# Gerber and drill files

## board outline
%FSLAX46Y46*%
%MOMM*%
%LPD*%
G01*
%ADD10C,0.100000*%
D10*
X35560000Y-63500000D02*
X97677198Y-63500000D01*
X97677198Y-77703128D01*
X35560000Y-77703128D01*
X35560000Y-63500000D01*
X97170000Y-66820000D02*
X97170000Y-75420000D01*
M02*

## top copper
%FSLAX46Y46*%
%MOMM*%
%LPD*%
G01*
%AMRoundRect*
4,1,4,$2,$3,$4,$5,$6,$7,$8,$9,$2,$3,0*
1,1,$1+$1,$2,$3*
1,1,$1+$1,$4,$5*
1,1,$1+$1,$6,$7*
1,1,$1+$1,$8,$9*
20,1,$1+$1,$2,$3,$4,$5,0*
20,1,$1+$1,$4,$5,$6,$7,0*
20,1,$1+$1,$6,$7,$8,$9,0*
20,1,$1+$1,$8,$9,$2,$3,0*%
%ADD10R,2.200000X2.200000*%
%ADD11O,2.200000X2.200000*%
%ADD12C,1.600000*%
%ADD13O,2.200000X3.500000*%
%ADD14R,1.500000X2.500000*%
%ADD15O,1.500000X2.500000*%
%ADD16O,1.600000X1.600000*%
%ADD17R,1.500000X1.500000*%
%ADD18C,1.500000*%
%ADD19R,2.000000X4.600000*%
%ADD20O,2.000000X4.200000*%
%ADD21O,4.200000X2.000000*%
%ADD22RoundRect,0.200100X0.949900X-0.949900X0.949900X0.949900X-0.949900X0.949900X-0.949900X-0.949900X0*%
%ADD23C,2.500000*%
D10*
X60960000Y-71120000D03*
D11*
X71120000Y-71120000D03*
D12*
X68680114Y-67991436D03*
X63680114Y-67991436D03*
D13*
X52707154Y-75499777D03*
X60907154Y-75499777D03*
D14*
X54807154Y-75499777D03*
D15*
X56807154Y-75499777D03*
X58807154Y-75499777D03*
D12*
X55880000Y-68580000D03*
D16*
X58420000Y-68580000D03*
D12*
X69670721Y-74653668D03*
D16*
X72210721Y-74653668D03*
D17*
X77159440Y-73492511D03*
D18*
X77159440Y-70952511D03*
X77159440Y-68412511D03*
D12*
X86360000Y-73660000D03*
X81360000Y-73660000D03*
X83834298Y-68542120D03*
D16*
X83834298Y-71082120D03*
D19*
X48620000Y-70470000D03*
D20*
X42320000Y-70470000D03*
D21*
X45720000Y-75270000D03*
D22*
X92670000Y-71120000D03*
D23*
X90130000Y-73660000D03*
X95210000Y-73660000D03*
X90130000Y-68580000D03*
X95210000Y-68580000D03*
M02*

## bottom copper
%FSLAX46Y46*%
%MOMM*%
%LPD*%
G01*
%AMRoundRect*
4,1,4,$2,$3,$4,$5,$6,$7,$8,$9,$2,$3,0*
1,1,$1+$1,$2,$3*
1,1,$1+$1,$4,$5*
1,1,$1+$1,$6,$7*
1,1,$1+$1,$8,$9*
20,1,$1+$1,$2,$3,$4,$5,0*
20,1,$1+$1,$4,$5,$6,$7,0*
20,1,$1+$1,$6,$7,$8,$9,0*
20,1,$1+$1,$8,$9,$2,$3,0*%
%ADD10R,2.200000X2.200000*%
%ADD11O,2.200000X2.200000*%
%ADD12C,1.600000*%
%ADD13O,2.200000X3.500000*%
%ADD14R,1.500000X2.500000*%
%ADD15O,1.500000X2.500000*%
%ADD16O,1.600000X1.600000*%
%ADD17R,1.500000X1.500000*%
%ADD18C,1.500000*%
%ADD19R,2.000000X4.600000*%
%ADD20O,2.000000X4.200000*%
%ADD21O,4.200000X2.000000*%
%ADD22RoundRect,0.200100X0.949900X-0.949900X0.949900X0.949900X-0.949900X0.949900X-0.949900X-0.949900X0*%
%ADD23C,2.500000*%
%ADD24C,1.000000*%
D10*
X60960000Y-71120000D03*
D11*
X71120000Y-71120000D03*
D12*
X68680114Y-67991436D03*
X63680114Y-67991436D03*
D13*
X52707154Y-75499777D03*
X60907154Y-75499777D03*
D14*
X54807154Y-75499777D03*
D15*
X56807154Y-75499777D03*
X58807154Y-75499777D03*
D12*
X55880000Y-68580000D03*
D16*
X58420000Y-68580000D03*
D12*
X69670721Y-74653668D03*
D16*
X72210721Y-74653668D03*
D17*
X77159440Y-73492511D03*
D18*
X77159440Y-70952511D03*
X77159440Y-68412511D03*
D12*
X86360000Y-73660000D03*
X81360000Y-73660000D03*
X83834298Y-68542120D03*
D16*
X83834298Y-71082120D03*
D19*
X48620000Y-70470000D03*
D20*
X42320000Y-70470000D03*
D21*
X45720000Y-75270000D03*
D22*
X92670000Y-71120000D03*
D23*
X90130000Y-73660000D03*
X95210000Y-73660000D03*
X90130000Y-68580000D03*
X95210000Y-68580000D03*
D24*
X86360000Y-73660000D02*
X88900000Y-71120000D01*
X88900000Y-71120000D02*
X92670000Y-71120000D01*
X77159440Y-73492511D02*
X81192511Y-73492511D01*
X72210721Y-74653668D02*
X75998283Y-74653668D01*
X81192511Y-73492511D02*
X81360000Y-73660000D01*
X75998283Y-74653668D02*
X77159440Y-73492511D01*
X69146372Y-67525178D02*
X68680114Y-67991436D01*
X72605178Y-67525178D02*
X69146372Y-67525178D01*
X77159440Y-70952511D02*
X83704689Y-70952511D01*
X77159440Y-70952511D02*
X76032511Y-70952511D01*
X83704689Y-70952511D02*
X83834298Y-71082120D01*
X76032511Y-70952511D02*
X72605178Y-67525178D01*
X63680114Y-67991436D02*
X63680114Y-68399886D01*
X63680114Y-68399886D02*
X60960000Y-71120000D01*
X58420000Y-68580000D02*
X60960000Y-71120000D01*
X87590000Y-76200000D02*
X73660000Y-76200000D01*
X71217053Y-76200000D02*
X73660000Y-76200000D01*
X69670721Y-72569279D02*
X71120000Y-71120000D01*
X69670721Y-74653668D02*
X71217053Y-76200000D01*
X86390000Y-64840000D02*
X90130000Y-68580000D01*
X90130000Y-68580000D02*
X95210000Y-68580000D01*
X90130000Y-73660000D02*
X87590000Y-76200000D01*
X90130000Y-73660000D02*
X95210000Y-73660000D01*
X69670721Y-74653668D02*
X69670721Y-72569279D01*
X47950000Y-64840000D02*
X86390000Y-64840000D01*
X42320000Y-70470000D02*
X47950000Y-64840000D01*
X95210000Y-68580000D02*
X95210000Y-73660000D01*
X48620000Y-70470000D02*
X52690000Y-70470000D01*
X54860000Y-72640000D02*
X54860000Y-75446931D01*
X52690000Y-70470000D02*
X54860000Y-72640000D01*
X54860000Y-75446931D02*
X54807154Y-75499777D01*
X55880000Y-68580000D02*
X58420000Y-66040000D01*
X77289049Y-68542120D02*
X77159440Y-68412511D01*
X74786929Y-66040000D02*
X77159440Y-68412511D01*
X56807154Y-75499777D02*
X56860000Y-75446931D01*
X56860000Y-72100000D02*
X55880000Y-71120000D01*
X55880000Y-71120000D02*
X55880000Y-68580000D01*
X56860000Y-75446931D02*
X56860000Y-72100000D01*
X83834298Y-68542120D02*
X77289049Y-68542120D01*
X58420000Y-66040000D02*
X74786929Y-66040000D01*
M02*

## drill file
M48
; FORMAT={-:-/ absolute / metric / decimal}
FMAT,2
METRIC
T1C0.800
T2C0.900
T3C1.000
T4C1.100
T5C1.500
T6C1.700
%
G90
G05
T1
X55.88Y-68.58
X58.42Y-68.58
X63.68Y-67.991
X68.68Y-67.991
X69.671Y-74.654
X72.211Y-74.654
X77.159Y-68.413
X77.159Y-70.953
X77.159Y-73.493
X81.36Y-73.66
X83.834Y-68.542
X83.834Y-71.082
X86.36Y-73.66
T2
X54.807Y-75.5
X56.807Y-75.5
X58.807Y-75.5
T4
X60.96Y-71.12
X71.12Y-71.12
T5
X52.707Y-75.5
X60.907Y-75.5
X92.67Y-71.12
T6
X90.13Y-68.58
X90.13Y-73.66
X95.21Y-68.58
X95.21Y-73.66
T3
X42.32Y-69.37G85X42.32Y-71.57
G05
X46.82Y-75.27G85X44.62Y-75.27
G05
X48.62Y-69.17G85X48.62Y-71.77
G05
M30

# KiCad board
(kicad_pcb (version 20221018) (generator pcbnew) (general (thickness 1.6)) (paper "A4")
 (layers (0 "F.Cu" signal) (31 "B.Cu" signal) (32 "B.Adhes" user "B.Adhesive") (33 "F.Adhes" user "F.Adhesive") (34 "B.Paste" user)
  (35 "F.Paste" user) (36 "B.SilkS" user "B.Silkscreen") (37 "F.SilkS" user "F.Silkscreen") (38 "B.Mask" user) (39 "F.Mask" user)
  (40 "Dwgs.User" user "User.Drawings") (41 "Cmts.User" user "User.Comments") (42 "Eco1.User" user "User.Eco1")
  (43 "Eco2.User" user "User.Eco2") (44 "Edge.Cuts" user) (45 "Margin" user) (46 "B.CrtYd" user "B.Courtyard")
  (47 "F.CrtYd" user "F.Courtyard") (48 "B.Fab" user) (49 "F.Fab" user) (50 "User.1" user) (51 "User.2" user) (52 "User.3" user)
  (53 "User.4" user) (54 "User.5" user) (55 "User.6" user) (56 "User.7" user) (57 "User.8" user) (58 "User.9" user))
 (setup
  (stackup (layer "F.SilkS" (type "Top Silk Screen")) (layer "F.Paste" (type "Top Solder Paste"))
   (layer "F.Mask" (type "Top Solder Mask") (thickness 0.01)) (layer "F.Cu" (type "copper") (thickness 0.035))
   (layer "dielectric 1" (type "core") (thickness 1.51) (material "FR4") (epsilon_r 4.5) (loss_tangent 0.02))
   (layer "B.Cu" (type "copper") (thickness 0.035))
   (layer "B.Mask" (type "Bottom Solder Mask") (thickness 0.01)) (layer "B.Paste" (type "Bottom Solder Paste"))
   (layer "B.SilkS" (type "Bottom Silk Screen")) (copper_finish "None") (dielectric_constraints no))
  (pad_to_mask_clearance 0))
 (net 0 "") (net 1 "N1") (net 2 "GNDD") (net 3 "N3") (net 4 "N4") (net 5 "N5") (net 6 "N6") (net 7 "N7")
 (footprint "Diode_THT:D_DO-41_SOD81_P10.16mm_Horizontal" (layer "F.Cu") (at 60.96 71.12)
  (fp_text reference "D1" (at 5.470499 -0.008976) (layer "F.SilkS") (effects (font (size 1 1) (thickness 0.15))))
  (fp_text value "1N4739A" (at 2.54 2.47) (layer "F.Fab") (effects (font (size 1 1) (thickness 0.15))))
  (pad "1" thru_hole rect (at 0 0) (size 2.2 2.2) (drill 1.1) (layers "*.Cu" "*.Mask") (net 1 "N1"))
  (pad "2" thru_hole oval (at 10.16 0) (size 2.2 2.2) (drill 1.1) (layers "*.Cu" "*.Mask") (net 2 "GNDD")))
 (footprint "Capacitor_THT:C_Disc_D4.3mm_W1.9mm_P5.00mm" (layer "F.Cu") (at 68.680114 67.991436 180)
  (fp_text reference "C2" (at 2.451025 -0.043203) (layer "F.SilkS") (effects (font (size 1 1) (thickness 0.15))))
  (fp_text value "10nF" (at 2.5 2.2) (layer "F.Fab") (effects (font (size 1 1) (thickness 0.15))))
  (pad "1" thru_hole circle (at 0 0 180) (size 1.6 1.6) (drill 0.8) (layers "*.Cu" "*.Mask") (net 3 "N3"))
  (pad "2" thru_hole circle (at 5 0 180) (size 1.6 1.6) (drill 0.8) (layers "*.Cu" "*.Mask") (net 1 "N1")))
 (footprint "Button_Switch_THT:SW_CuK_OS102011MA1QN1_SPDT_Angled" (layer "F.Cu") (at 54.807154 75.499777)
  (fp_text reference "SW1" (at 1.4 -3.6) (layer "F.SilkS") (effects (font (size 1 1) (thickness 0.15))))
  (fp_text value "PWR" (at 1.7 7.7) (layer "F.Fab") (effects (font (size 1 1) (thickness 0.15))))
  (pad "" thru_hole oval (at -2.1 0) (size 2.2 3.5) (drill 1.5) (layers "*.Cu" "*.Mask"))
  (pad "" thru_hole oval (at 6.1 0) (size 2.2 3.5) (drill 1.5) (layers "*.Cu" "*.Mask"))
  (pad "1" thru_hole rect (at 0 0) (size 1.5 2.5) (drill 0.9) (layers "*.Cu" "*.Mask") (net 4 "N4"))
  (pad "2" thru_hole oval (at 2 0) (size 1.5 2.5) (drill 0.9) (layers "*.Cu" "*.Mask") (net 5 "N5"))
  (pad "3" thru_hole oval (at 4 0) (size 1.5 2.5) (drill 0.9) (layers "*.Cu" "*.Mask")))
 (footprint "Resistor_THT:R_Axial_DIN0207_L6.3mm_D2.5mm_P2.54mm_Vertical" (layer "F.Cu") (at 55.88 68.58)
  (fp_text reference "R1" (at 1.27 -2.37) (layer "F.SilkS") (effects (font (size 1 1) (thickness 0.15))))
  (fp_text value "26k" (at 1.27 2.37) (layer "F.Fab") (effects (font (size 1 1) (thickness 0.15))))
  (pad "1" thru_hole circle (at 0 0) (size 1.6 1.6) (drill 0.8) (layers "*.Cu" "*.Mask") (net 5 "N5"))
  (pad "2" thru_hole oval (at 2.54 0) (size 1.6 1.6) (drill 0.8) (layers "*.Cu" "*.Mask") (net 1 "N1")))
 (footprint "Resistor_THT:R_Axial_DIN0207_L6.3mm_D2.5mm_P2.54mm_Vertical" (layer "F.Cu") (at 69.670721 74.653668)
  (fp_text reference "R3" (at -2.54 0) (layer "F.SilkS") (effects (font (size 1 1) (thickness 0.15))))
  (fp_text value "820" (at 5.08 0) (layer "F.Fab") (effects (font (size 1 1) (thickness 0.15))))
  (pad "1" thru_hole circle (at 0 0) (size 1.6 1.6) (drill 0.8) (layers "*.Cu" "*.Mask") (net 2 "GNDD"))
  (pad "2" thru_hole oval (at 2.54 0) (size 1.6 1.6) (drill 0.8) (layers "*.Cu" "*.Mask") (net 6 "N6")))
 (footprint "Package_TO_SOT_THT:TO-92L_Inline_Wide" (layer "F.Cu") (at 77.15944 73.492511 90)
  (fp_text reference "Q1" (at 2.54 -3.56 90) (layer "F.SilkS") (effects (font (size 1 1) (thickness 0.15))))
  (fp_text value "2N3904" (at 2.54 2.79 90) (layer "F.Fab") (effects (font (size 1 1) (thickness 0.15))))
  (pad "1" thru_hole rect (at 0 0 90) (size 1.5 1.5) (drill 0.8) (layers "*.Cu" "*.Mask") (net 6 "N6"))
  (pad "2" thru_hole circle (at 2.54 0 90) (size 1.5 1.5) (drill 0.8) (layers "*.Cu" "*.Mask") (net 3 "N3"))
  (pad "3" thru_hole circle (at 5.08 0 90) (size 1.5 1.5) (drill 0.8) (layers "*.Cu" "*.Mask") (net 5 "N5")))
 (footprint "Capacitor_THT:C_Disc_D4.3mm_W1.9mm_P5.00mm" (layer "F.Cu") (at 86.36 73.66 180)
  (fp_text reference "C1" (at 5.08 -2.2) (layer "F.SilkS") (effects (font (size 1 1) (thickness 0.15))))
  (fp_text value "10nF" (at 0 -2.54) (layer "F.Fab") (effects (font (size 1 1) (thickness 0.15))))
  (pad "1" thru_hole circle (at 0 0 180) (size 1.6 1.6) (drill 0.8) (layers "*.Cu" "*.Mask") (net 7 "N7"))
  (pad "2" thru_hole circle (at 5 0 180) (size 1.6 1.6) (drill 0.8) (layers "*.Cu" "*.Mask") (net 6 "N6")))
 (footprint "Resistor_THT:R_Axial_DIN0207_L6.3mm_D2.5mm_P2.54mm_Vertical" (layer "F.Cu") (at 83.834298 68.54212 -90)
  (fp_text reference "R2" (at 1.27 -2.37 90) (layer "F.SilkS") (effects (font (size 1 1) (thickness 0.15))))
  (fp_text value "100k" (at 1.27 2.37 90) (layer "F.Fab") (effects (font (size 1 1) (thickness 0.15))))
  (pad "1" thru_hole circle (at 0 0 270) (size 1.6 1.6) (drill 0.8) (layers "*.Cu" "*.Mask") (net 5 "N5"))
  (pad "2" thru_hole oval (at 2.54 0 270) (size 1.6 1.6) (drill 0.8) (layers "*.Cu" "*.Mask") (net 3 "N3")))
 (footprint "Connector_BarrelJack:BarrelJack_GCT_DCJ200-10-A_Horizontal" (layer "F.Cu") (at 48.62 70.47 -90)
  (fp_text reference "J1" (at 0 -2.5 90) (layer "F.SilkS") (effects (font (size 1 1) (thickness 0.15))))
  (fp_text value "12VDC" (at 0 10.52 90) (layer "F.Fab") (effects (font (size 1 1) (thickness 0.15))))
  (pad "1" thru_hole rect (at 0 0 270) (size 4.6 2) (drill oval 3.6 1) (layers "*.Cu" "*.Mask") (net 4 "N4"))
  (pad "2" thru_hole oval (at 0 6.3 270) (size 4.2 2) (drill oval 3.2 1) (layers "*.Cu" "*.Mask") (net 2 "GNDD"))
  (pad "3" thru_hole oval (at 4.8 2.9 270) (size 2 4.2) (drill oval 1 3.2) (layers "*.Cu" "*.Mask")))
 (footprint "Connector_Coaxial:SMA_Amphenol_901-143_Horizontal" (layer "B.Cu") (at 92.67 71.12 90)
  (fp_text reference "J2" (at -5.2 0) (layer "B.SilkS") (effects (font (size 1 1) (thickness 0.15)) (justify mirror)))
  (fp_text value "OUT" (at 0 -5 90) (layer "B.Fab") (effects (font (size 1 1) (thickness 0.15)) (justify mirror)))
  (fp_line (start 4.3 4.5) (end -4.3 4.5) (stroke (width 0.1) (type solid)) (layer "Edge.Cuts"))
  (pad "1" thru_hole roundrect (at 0 0 90) (size 2.3 2.3) (drill 1.5) (layers "*.Cu" "*.Mask") (remove_unused_layers) (keep_end_layers)
   (zone_layer_connections) (roundrect_rratio 0.087) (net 7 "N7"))
  (pad "2" thru_hole circle (at -2.54 -2.54 90) (size 2.5 2.5) (drill 1.7) (layers "*.Cu" "*.Mask") (remove_unused_layers) (keep_end_layers)
   (zone_layer_connections) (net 2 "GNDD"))
  (pad "2" thru_hole circle (at -2.54 2.54 90) (size 2.5 2.5) (drill 1.7) (layers "*.Cu" "*.Mask") (remove_unused_layers) (keep_end_layers)
   (zone_layer_connections) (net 2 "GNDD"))
  (pad "2" thru_hole circle (at 2.54 -2.54 90) (size 2.5 2.5) (drill 1.7) (layers "*.Cu" "*.Mask") (remove_unused_layers) (keep_end_layers)
   (zone_layer_connections) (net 2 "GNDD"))
  (pad "2" thru_hole circle (at 2.54 2.54 90) (size 2.5 2.5) (drill 1.7) (layers "*.Cu" "*.Mask") (remove_unused_layers) (keep_end_layers)
   (zone_layer_connections) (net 2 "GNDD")))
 (gr_rect (start 35.56 63.5) (end 97.677198 77.703128) (stroke (width 0.1) (type default)) (fill none) (layer "Edge.Cuts"))
 (segment (start 86.36 73.66) (end 88.9 71.12) (width 1) (layer "B.Cu") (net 7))
 (segment (start 88.9 71.12) (end 92.67 71.12) (width 1) (layer "B.Cu") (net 7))
 (segment (start 77.15944 73.492511) (end 81.192511 73.492511) (width 1) (layer "B.Cu") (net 6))
 (segment (start 72.210721 74.653668) (end 75.998283 74.653668) (width 1) (layer "B.Cu") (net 6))
 (segment (start 81.192511 73.492511) (end 81.36 73.66) (width 1) (layer "B.Cu") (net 6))
 (segment (start 75.998283 74.653668) (end 77.15944 73.492511) (width 1) (layer "B.Cu") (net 6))
 (segment (start 69.146372 67.525178) (end 68.680114 67.991436) (width 1) (layer "B.Cu") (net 3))
 (segment (start 72.605178 67.525178) (end 69.146372 67.525178) (width 1) (layer "B.Cu") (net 3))
 (segment (start 77.15944 70.952511) (end 83.704689 70.952511) (width 1) (layer "B.Cu") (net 3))
 (segment (start 77.15944 70.952511) (end 76.032511 70.952511) (width 1) (layer "B.Cu") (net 3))
 (segment (start 83.704689 70.952511) (end 83.834298 71.08212) (width 1) (layer "B.Cu") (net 3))
 (segment (start 76.032511 70.952511) (end 72.605178 67.525178) (width 1) (layer "B.Cu") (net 3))
 (segment (start 63.680114 67.991436) (end 63.680114 68.399886) (width 1) (layer "B.Cu") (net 1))
 (segment (start 63.680114 68.399886) (end 60.96 71.12) (width 1) (layer "B.Cu") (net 1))
 (segment (start 58.42 68.58) (end 60.96 71.12) (width 1) (layer "B.Cu") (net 1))
 (segment (start 87.59 76.2) (end 73.66 76.2) (width 1) (layer "B.Cu") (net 2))
 (segment (start 71.217053 76.2) (end 73.66 76.2) (width 1) (layer "B.Cu") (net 2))
 (segment (start 69.670721 72.569279) (end 71.12 71.12) (width 1) (layer "B.Cu") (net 2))
 (segment (start 69.670721 74.653668) (end 71.217053 76.2) (width 1) (layer "B.Cu") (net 2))
 (segment (start 86.39 64.84) (end 90.13 68.58) (width 1) (layer "B.Cu") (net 2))
 (segment (start 90.13 68.58) (end 95.21 68.58) (width 1) (layer "B.Cu") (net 2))
 (segment (start 90.13 73.66) (end 87.59 76.2) (width 1) (layer "B.Cu") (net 2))
 (segment (start 90.13 73.66) (end 95.21 73.66) (width 1) (layer "B.Cu") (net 2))
 (segment (start 69.670721 74.653668) (end 69.670721 72.569279) (width 1) (layer "B.Cu") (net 2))
 (segment (start 47.95 64.84) (end 86.39 64.84) (width 1) (layer "B.Cu") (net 2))
 (segment (start 42.32 70.47) (end 47.95 64.84) (width 1) (layer "B.Cu") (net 2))
 (segment (start 95.21 68.58) (end 95.21 73.66) (width 1) (layer "B.Cu") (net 2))
 (segment (start 48.62 70.47) (end 52.69 70.47) (width 1) (layer "B.Cu") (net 4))
 (segment (start 54.86 72.64) (end 54.86 75.446931) (width 1) (layer "B.Cu") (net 4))
 (segment (start 52.69 70.47) (end 54.86 72.64) (width 1) (layer "B.Cu") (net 4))
 (segment (start 54.86 75.446931) (end 54.807154 75.499777) (width 1) (layer "B.Cu") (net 4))
 (segment (start 55.88 68.58) (end 58.42 66.04) (width 1) (layer "B.Cu") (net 5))
 (segment (start 77.289049 68.54212) (end 77.15944 68.412511) (width 1) (layer "B.Cu") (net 5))
 (segment (start 74.786929 66.04) (end 77.15944 68.412511) (width 1) (layer "B.Cu") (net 5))
 (segment (start 56.807154 75.499777) (end 56.86 75.446931) (width 1) (layer "B.Cu") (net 5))
 (segment (start 56.86 72.1) (end 55.88 71.12) (width 1) (layer "B.Cu") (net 5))
 (segment (start 55.88 71.12) (end 55.88 68.58) (width 1) (layer "B.Cu") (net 5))
 (segment (start 56.86 75.446931) (end 56.86 72.1) (width 1) (layer "B.Cu") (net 5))
 (segment (start 83.834298 68.54212) (end 77.289049 68.54212) (width 1) (layer "B.Cu") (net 5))
 (segment (start 58.42 66.04) (end 74.786929 66.04) (width 1) (layer "B.Cu") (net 5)))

